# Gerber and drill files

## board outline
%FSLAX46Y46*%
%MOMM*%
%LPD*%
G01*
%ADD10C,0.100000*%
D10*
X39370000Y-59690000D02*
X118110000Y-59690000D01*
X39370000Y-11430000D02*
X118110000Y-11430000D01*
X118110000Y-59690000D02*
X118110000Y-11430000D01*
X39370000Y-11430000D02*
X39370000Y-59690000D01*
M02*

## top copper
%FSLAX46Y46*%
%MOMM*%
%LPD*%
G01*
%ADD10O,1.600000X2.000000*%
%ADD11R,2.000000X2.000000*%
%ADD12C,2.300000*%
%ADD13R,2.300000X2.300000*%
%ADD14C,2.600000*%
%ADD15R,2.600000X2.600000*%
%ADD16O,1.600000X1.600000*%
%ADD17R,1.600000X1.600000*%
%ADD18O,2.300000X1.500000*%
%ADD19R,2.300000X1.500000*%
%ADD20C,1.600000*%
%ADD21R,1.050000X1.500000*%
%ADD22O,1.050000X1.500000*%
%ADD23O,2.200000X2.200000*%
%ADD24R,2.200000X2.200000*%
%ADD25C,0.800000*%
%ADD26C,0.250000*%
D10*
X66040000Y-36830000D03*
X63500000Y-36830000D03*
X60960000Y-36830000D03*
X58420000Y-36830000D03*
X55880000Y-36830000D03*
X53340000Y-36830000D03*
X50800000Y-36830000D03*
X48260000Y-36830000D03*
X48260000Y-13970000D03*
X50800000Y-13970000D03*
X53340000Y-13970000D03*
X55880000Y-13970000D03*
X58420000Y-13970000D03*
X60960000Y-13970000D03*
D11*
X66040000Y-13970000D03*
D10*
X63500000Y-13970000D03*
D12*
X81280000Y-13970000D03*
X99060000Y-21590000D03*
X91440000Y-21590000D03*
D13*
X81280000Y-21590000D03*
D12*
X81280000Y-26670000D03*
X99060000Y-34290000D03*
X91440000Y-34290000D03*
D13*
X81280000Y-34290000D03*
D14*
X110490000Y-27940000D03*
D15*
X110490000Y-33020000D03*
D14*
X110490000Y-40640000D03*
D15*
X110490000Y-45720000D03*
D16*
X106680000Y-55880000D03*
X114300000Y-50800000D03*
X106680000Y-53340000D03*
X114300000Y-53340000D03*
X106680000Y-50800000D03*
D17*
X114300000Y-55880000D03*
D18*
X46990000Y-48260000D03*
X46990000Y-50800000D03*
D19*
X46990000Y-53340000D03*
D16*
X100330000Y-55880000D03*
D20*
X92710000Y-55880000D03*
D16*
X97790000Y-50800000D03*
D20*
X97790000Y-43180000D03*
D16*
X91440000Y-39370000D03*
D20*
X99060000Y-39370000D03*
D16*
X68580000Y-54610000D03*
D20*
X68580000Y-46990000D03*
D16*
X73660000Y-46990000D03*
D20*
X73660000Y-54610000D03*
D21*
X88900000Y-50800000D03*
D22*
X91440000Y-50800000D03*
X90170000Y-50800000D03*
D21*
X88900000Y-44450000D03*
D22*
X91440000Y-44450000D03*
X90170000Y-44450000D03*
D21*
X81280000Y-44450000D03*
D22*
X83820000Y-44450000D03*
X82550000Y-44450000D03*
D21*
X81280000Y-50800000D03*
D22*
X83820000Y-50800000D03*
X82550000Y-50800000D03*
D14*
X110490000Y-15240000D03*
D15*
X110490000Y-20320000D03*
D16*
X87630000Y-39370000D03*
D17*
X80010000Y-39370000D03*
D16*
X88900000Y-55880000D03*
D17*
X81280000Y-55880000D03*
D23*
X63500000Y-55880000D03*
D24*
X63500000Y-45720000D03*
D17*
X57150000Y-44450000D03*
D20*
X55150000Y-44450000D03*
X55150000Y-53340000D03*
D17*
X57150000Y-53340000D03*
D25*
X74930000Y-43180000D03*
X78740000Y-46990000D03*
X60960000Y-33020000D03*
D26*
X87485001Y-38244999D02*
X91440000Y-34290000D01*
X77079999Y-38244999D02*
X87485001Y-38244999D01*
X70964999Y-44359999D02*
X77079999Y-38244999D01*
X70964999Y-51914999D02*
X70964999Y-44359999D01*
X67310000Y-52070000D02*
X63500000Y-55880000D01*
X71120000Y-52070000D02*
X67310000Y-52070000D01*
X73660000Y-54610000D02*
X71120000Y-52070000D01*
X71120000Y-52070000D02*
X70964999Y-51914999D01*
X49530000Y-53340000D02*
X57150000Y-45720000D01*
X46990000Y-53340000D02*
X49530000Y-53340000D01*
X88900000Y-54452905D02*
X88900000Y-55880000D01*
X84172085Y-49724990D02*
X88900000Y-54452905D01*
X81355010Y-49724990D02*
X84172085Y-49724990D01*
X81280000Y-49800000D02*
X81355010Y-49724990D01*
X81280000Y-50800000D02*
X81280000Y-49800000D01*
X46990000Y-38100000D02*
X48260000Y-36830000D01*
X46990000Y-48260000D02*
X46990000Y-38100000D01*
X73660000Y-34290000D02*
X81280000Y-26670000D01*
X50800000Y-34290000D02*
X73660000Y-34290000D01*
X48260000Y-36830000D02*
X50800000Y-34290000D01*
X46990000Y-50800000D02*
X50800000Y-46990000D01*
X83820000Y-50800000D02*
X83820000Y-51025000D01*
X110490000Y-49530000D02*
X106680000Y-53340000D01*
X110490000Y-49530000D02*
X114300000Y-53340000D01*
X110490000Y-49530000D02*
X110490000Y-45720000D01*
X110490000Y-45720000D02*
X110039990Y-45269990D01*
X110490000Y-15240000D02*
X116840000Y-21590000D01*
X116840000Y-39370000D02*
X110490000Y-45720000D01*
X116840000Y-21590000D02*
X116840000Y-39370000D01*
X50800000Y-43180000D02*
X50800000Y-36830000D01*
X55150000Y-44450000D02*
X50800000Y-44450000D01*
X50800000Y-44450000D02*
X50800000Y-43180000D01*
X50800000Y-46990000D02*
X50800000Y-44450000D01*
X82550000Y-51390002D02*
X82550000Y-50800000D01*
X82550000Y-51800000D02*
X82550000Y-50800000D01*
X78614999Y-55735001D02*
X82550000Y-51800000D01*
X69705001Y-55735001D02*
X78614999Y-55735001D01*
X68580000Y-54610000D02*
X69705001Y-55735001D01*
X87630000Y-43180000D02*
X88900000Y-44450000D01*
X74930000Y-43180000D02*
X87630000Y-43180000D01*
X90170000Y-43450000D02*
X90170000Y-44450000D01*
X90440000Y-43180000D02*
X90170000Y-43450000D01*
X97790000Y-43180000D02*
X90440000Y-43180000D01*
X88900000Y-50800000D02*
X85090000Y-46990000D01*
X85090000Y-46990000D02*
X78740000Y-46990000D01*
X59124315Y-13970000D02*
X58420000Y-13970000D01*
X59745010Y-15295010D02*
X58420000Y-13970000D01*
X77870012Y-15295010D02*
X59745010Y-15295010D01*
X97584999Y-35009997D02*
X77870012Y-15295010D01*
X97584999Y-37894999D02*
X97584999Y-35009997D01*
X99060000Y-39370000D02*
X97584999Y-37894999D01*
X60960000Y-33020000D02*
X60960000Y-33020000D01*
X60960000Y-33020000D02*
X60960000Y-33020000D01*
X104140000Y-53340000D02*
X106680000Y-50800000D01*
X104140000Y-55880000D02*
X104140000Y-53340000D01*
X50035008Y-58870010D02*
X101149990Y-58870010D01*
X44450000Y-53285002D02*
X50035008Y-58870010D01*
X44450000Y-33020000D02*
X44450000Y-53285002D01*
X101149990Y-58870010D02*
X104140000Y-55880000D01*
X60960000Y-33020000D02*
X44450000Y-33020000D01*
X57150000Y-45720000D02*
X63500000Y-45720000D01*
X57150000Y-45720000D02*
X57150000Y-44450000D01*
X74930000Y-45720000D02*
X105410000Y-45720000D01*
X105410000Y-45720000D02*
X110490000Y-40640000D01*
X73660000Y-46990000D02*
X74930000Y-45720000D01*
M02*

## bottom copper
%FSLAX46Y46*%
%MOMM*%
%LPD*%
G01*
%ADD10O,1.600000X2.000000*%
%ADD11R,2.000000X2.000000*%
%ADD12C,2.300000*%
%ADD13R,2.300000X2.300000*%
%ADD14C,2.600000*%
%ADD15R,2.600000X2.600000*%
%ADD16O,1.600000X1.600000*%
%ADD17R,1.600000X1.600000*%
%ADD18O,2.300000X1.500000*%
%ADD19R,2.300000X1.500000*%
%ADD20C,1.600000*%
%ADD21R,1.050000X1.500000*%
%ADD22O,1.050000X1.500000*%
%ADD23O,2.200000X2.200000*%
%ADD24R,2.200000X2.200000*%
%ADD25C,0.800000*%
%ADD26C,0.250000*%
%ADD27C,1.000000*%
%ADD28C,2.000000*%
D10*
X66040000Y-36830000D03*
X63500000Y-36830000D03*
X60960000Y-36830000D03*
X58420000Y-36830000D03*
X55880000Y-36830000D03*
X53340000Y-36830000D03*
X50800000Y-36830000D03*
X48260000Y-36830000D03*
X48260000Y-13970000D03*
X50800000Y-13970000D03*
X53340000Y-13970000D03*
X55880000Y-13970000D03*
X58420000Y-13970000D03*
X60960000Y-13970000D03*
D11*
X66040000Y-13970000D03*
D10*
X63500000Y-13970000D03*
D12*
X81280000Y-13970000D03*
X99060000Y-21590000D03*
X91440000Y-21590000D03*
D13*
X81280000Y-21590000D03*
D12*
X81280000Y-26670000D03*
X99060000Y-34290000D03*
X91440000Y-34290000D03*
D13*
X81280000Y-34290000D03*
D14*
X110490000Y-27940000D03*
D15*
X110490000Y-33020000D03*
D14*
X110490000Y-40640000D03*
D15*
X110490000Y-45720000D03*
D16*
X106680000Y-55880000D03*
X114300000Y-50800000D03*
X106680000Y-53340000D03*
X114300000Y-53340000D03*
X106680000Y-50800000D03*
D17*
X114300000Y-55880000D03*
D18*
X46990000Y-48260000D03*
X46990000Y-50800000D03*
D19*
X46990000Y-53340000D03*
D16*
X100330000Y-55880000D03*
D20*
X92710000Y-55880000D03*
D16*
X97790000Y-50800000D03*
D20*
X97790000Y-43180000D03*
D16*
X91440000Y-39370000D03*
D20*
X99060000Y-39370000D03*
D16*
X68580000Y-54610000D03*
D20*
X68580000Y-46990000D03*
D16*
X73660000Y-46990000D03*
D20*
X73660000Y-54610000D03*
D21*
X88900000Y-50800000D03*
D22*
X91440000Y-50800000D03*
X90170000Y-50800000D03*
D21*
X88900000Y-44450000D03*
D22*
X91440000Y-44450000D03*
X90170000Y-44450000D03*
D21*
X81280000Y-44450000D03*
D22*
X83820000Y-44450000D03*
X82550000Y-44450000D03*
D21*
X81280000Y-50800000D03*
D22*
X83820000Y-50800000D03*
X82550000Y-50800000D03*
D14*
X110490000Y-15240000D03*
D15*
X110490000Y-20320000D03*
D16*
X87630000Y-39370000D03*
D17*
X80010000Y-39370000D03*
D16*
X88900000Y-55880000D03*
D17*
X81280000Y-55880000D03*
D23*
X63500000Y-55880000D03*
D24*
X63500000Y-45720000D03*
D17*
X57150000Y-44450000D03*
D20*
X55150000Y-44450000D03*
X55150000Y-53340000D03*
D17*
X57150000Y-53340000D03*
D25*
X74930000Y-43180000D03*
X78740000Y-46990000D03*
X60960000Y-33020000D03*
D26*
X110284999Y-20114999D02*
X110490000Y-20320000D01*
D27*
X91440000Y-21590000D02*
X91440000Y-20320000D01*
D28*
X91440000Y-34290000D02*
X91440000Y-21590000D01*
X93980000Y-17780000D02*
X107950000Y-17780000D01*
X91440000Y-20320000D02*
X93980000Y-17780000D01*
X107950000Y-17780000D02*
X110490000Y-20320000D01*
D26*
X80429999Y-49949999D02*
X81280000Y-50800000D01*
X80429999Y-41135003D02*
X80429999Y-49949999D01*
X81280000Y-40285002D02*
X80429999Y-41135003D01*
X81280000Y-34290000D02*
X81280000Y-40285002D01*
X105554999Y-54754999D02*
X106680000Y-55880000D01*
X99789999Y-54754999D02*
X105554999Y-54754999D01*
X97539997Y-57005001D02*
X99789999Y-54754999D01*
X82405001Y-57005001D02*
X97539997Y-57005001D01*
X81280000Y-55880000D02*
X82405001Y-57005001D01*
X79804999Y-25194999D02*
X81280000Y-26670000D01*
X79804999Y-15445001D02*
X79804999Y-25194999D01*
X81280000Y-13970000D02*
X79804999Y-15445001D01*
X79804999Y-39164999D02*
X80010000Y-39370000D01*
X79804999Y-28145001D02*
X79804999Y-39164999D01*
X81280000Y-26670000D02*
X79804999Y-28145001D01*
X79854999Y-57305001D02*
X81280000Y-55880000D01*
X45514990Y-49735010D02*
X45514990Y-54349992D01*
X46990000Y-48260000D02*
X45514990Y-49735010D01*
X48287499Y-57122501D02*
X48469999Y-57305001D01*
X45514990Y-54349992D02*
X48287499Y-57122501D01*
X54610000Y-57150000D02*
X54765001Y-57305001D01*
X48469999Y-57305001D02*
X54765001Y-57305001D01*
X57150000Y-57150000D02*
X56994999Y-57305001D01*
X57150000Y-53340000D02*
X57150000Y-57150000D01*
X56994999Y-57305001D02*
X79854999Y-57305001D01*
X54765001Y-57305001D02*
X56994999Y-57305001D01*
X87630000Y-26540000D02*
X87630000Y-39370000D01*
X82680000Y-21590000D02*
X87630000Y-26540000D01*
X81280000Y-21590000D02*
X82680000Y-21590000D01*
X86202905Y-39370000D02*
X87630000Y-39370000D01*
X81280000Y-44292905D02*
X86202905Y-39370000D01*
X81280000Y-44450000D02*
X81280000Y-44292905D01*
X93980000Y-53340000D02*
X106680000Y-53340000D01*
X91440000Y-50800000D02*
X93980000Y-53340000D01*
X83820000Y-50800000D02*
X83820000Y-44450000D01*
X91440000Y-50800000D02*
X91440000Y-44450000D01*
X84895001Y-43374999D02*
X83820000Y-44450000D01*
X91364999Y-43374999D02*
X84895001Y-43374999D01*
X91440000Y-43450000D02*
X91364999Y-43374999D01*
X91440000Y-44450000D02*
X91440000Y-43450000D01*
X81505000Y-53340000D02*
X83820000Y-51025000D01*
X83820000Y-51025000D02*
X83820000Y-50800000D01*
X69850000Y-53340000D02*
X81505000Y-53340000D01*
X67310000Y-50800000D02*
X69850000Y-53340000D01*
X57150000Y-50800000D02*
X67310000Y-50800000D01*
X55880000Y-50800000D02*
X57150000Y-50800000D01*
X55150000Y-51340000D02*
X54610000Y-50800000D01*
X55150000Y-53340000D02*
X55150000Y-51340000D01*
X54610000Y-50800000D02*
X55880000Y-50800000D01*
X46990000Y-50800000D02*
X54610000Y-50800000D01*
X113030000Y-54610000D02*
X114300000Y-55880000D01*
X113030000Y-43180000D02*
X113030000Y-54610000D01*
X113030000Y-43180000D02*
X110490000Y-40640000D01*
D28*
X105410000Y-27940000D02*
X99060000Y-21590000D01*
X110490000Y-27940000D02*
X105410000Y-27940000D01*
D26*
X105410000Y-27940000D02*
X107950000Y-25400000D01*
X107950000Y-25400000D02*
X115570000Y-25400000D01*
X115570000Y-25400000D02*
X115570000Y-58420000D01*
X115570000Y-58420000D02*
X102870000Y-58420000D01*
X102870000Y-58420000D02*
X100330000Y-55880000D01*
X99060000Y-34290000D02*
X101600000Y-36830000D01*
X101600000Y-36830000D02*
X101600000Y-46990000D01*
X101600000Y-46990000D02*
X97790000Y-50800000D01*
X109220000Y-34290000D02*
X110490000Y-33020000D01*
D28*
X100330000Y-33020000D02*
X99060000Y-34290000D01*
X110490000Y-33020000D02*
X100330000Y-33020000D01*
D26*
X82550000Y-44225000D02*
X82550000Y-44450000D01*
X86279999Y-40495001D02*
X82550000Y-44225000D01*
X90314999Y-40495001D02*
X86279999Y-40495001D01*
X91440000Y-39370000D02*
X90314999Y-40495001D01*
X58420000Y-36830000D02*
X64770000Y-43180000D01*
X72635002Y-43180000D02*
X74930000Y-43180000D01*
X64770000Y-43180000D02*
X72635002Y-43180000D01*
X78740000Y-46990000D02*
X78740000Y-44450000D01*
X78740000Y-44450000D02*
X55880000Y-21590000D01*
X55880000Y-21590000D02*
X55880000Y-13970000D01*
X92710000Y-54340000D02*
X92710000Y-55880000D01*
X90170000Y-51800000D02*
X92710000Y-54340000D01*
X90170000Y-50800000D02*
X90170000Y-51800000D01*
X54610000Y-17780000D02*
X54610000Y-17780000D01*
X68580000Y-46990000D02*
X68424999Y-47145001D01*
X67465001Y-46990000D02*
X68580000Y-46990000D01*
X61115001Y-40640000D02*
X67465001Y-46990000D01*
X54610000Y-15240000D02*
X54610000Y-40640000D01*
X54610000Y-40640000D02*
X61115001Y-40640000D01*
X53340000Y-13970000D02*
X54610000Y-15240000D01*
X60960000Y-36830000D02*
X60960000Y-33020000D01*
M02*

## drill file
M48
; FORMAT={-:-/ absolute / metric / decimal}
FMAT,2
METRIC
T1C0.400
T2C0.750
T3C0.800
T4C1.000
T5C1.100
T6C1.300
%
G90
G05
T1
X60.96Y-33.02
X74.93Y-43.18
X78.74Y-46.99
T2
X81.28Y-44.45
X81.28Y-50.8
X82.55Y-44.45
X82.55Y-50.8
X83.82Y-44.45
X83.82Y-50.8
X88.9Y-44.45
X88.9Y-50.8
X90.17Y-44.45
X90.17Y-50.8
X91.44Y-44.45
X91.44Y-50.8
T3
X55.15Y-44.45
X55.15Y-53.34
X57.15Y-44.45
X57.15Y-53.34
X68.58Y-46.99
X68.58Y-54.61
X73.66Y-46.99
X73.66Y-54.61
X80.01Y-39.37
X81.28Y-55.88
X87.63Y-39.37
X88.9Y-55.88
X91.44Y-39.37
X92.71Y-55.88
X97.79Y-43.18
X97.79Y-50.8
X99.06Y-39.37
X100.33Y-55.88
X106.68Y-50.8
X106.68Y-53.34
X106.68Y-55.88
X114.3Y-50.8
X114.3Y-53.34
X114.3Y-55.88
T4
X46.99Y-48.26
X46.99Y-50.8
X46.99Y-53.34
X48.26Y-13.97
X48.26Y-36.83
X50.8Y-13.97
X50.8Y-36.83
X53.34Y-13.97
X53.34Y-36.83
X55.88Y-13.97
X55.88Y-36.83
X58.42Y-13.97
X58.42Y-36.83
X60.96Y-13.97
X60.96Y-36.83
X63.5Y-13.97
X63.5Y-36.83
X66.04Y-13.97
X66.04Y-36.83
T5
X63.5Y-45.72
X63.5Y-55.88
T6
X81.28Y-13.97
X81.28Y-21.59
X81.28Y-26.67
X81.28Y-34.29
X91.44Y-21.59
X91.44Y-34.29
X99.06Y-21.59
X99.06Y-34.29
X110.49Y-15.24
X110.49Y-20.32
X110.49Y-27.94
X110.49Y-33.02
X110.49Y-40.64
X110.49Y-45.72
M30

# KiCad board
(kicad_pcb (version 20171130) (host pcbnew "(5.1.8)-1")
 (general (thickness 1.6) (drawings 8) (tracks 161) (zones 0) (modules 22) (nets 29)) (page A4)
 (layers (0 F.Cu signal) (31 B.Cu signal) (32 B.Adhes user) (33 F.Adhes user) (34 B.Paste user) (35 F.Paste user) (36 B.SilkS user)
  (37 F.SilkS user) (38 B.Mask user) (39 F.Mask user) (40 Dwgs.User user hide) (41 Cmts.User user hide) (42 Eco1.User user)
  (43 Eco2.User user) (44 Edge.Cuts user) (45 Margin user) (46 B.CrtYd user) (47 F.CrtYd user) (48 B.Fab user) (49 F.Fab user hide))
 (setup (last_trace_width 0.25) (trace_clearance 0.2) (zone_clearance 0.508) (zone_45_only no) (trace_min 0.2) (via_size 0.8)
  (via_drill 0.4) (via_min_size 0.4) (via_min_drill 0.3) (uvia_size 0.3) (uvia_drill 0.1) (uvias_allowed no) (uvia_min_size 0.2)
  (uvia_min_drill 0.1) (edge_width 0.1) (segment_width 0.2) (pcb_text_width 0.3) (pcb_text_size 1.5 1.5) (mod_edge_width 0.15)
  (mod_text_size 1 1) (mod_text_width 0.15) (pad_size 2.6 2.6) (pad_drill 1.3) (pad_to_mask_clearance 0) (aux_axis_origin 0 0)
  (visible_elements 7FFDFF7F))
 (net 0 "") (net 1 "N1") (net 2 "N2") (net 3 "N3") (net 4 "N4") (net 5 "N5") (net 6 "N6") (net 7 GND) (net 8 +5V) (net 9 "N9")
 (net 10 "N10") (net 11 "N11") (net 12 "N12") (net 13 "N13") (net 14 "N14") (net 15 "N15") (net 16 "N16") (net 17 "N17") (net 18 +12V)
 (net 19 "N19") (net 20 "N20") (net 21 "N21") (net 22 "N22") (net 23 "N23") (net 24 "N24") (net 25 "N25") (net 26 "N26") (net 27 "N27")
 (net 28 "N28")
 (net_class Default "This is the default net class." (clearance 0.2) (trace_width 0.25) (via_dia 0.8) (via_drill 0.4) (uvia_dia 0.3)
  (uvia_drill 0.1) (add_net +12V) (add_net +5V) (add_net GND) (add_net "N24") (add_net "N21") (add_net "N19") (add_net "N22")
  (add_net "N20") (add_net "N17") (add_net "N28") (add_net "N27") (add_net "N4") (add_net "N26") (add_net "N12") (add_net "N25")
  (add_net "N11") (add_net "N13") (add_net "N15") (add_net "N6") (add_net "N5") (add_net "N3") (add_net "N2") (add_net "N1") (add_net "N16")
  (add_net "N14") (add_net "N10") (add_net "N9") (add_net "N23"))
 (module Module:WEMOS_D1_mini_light (layer F.Cu) (at 66.04 13.97 270)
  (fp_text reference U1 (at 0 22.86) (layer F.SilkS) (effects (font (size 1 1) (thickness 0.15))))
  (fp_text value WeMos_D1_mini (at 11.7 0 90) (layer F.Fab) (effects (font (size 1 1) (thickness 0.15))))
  (pad 16 thru_hole oval (at 22.86 0 270) (size 2 1.6) (drill 1) (layers *.Cu *.Mask) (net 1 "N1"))
  (pad 15 thru_hole oval (at 22.86 2.54 270) (size 2 1.6) (drill 1) (layers *.Cu *.Mask) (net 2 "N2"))
  (pad 14 thru_hole oval (at 22.86 5.08 270) (size 2 1.6) (drill 1) (layers *.Cu *.Mask) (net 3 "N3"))
  (pad 13 thru_hole oval (at 22.86 7.62 270) (size 2 1.6) (drill 1) (layers *.Cu *.Mask) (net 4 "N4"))
  (pad 12 thru_hole oval (at 22.86 10.16 270) (size 2 1.6) (drill 1) (layers *.Cu *.Mask) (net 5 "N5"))
  (pad 11 thru_hole oval (at 22.86 12.7 270) (size 2 1.6) (drill 1) (layers *.Cu *.Mask) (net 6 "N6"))
  (pad 10 thru_hole oval (at 22.86 15.24 270) (size 2 1.6) (drill 1) (layers *.Cu *.Mask) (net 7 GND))
  (pad 9 thru_hole oval (at 22.86 17.78 270) (size 2 1.6) (drill 1) (layers *.Cu *.Mask) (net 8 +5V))
  (pad 8 thru_hole oval (at 0 17.78 270) (size 2 1.6) (drill 1) (layers *.Cu *.Mask) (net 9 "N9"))
  (pad 7 thru_hole oval (at 0 15.24 270) (size 2 1.6) (drill 1) (layers *.Cu *.Mask) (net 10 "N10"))
  (pad 6 thru_hole oval (at 0 12.7 270) (size 2 1.6) (drill 1) (layers *.Cu *.Mask) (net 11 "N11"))
  (pad 5 thru_hole oval (at 0 10.16 270) (size 2 1.6) (drill 1) (layers *.Cu *.Mask) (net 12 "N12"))
  (pad 4 thru_hole oval (at 0 7.62 270) (size 2 1.6) (drill 1) (layers *.Cu *.Mask) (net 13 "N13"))
  (pad 3 thru_hole oval (at 0 5.08 270) (size 2 1.6) (drill 1) (layers *.Cu *.Mask) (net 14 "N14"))
  (pad 1 thru_hole rect (at 0 0 270) (size 2 2) (drill 1) (layers *.Cu *.Mask) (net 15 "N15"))
  (pad 2 thru_hole oval (at 0 2.54 270) (size 2 1.6) (drill 1) (layers *.Cu *.Mask) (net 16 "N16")))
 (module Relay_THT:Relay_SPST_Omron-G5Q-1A (layer F.Cu) (at 81.28 21.59)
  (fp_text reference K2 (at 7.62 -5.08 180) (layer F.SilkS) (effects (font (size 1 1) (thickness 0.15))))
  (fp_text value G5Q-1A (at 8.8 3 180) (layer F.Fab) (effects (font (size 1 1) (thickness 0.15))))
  (pad 5 thru_hole circle (at 0 -7.62 180) (size 2.3 2.3) (drill 1.3) (layers *.Cu *.Mask) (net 8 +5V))
  (pad 3 thru_hole circle (at 17.78 0 180) (size 2.3 2.3) (drill 1.3) (layers *.Cu *.Mask) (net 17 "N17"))
  (pad 2 thru_hole circle (at 10.16 0 180) (size 2.3 2.3) (drill 1.3) (layers *.Cu *.Mask) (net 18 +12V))
  (pad 1 thru_hole rect (at 0 0 180) (size 2.3 2.3) (drill 1.3) (layers *.Cu *.Mask) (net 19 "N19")))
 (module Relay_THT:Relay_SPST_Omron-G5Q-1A (layer F.Cu) (at 81.28 34.29)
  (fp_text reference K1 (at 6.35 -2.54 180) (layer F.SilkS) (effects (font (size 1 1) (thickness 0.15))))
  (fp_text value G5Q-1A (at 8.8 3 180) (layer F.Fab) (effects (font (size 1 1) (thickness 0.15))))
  (pad 5 thru_hole circle (at 0 -7.62 180) (size 2.3 2.3) (drill 1.3) (layers *.Cu *.Mask) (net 8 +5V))
  (pad 3 thru_hole circle (at 17.78 0 180) (size 2.3 2.3) (drill 1.3) (layers *.Cu *.Mask) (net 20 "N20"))
  (pad 2 thru_hole circle (at 10.16 0 180) (size 2.3 2.3) (drill 1.3) (layers *.Cu *.Mask) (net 18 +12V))
  (pad 1 thru_hole rect (at 0 0 180) (size 2.3 2.3) (drill 1.3) (layers *.Cu *.Mask) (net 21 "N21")))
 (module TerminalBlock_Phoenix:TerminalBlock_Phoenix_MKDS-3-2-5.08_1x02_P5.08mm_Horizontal (layer F.Cu) (at 110.49 33.02 90)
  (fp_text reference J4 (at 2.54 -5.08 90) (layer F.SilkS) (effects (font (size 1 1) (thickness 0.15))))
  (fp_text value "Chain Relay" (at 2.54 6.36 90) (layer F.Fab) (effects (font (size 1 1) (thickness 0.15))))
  (pad 2 thru_hole circle (at 5.08 0 90) (size 2.6 2.6) (drill 1.3) (layers *.Cu *.Mask) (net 17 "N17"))
  (pad 1 thru_hole rect (at 0 0 90) (size 2.6 2.6) (drill 1.3) (layers *.Cu *.Mask) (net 20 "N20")))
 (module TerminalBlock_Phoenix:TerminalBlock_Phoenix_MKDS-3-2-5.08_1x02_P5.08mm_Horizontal (layer F.Cu) (at 110.49 45.72 90)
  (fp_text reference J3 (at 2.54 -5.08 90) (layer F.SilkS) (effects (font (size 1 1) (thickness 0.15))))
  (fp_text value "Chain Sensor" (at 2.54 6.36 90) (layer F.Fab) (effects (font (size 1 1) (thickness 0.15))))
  (pad 2 thru_hole circle (at 5.08 0 90) (size 2.6 2.6) (drill 1.3) (layers *.Cu *.Mask) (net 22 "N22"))
  (pad 1 thru_hole rect (at 0 0 90) (size 2.6 2.6) (drill 1.3) (layers *.Cu *.Mask) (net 7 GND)))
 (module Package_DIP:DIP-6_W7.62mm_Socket (layer F.Cu) (at 114.3 55.88 180)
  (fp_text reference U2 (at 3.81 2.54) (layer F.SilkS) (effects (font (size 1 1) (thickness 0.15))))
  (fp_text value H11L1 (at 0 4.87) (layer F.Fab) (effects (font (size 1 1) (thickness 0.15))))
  (pad 6 thru_hole oval (at 7.62 0 180) (size 1.6 1.6) (drill 0.8) (layers *.Cu *.Mask) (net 8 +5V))
  (pad 3 thru_hole oval (at 0 5.08 180) (size 1.6 1.6) (drill 0.8) (layers *.Cu *.Mask) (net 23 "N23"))
  (pad 5 thru_hole oval (at 7.62 2.54 180) (size 1.6 1.6) (drill 0.8) (layers *.Cu *.Mask) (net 7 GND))
  (pad 2 thru_hole oval (at 0 2.54 180) (size 1.6 1.6) (drill 0.8) (layers *.Cu *.Mask) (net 7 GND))
  (pad 4 thru_hole oval (at 7.62 5.08 180) (size 1.6 1.6) (drill 0.8) (layers *.Cu *.Mask) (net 3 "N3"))
  (pad 1 thru_hole rect (at 0 0 180) (size 1.6 1.6) (drill 0.8) (layers *.Cu *.Mask) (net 22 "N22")))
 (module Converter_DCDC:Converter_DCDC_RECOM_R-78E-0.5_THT (layer F.Cu) (at 46.99 53.34 90)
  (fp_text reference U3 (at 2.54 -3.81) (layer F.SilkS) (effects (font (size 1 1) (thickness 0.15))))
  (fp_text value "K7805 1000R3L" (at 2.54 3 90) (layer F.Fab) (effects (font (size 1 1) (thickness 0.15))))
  (pad 3 thru_hole oval (at 5.08 0 90) (size 1.5 2.3) (drill 1) (layers *.Cu *.Mask) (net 8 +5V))
  (pad 2 thru_hole oval (at 2.54 0 90) (size 1.5 2.3) (drill 1) (layers *.Cu *.Mask) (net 7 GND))
  (pad 1 thru_hole rect (at 0 0 90) (size 1.5 2.3) (drill 1) (layers *.Cu *.Mask) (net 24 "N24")))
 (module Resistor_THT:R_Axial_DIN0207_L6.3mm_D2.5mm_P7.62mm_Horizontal (layer F.Cu) (at 92.71 55.88)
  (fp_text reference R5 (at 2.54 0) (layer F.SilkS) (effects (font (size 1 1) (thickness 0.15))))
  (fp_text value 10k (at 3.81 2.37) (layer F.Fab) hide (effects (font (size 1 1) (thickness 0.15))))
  (pad 2 thru_hole oval (at 7.62 0) (size 1.6 1.6) (drill 0.8) (layers *.Cu *.Mask) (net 17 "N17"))
  (pad 1 thru_hole circle (at 0 0) (size 1.6 1.6) (drill 0.8) (layers *.Cu *.Mask) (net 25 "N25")))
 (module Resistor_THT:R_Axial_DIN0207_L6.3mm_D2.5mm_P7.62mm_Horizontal (layer F.Cu) (at 97.79 43.18 270)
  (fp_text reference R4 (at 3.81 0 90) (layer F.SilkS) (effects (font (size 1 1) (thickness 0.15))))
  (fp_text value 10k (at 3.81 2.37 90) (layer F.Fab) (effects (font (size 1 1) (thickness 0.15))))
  (pad 2 thru_hole oval (at 7.62 0 270) (size 1.6 1.6) (drill 0.8) (layers *.Cu *.Mask) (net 20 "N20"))
  (pad 1 thru_hole circle (at 0 0 270) (size 1.6 1.6) (drill 0.8) (layers *.Cu *.Mask) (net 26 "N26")))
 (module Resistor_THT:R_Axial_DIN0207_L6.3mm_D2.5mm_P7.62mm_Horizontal (layer F.Cu) (at 99.06 39.37 180)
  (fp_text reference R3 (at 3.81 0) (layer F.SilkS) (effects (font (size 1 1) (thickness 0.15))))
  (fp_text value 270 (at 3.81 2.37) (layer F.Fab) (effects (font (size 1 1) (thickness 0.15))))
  (pad 2 thru_hole oval (at 7.62 0 180) (size 1.6 1.6) (drill 0.8) (layers *.Cu *.Mask) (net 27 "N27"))
  (pad 1 thru_hole circle (at 0 0 180) (size 1.6 1.6) (drill 0.8) (layers *.Cu *.Mask) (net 13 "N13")))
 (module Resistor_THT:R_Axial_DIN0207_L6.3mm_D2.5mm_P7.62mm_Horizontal (layer F.Cu) (at 68.58 46.99 270)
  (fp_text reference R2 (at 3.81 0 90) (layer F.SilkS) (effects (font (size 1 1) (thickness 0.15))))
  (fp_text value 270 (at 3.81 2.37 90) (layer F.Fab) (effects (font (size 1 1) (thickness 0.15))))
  (pad 2 thru_hole oval (at 7.62 0 270) (size 1.6 1.6) (drill 0.8) (layers *.Cu *.Mask) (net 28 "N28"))
  (pad 1 thru_hole circle (at 0 0 270) (size 1.6 1.6) (drill 0.8) (layers *.Cu *.Mask) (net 11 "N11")))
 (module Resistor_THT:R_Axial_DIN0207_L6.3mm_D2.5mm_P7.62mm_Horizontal (layer F.Cu) (at 73.66 54.61 90)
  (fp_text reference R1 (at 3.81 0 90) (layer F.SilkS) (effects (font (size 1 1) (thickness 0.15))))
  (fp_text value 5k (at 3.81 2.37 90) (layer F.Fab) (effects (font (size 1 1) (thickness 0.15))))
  (pad 2 thru_hole oval (at 7.62 0 90) (size 1.6 1.6) (drill 0.8) (layers *.Cu *.Mask) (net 22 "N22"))
  (pad 1 thru_hole circle (at 0 0 90) (size 1.6 1.6) (drill 0.8) (layers *.Cu *.Mask) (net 18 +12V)))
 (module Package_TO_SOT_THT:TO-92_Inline (layer F.Cu) (at 88.9 50.8)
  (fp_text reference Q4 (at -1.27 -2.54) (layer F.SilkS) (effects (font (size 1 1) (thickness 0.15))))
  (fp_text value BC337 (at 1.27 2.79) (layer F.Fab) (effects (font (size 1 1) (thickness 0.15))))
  (pad 1 thru_hole rect (at 0 0) (size 1.05 1.5) (drill 0.75) (layers *.Cu *.Mask) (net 12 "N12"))
  (pad 3 thru_hole oval (at 2.54 0) (size 1.05 1.5) (drill 0.75) (layers *.Cu *.Mask) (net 7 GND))
  (pad 2 thru_hole oval (at 1.27 0) (size 1.05 1.5) (drill 0.75) (layers *.Cu *.Mask) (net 25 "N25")))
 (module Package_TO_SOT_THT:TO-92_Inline (layer F.Cu) (at 88.9 44.45)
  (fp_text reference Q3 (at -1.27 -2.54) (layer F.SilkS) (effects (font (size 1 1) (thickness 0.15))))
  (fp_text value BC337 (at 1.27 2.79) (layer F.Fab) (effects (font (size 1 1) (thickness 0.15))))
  (pad 1 thru_hole rect (at 0 0) (size 1.05 1.5) (drill 0.75) (layers *.Cu *.Mask) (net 4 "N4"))
  (pad 3 thru_hole oval (at 2.54 0) (size 1.05 1.5) (drill 0.75) (layers *.Cu *.Mask) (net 7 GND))
  (pad 2 thru_hole oval (at 1.27 0) (size 1.05 1.5) (drill 0.75) (layers *.Cu *.Mask) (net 26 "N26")))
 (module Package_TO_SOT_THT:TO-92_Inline (layer F.Cu) (at 81.28 44.45)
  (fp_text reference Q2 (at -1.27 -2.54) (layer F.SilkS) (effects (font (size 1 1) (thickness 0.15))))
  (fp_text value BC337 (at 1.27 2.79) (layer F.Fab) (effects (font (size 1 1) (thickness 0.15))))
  (pad 1 thru_hole rect (at 0 0) (size 1.05 1.5) (drill 0.75) (layers *.Cu *.Mask) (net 19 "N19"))
  (pad 3 thru_hole oval (at 2.54 0) (size 1.05 1.5) (drill 0.75) (layers *.Cu *.Mask) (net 7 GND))
  (pad 2 thru_hole oval (at 1.27 0) (size 1.05 1.5) (drill 0.75) (layers *.Cu *.Mask) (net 27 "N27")))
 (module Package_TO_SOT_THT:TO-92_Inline (layer F.Cu) (at 81.28 50.8)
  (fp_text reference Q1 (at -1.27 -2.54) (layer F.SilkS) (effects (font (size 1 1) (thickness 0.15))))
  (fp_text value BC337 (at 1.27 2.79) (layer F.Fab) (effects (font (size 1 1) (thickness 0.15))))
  (pad 1 thru_hole rect (at 0 0) (size 1.05 1.5) (drill 0.75) (layers *.Cu *.Mask) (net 21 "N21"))
  (pad 3 thru_hole oval (at 2.54 0) (size 1.05 1.5) (drill 0.75) (layers *.Cu *.Mask) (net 7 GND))
  (pad 2 thru_hole oval (at 1.27 0) (size 1.05 1.5) (drill 0.75) (layers *.Cu *.Mask) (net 28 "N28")))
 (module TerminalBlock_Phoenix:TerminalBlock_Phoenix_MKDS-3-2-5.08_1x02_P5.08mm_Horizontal (layer F.Cu) (at 110.49 20.32 90)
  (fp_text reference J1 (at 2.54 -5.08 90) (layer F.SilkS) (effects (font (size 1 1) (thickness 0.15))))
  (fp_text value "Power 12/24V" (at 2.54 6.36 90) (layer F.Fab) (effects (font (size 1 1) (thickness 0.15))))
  (pad 2 thru_hole circle (at 5.08 0 90) (size 2.6 2.6) (drill 1.3) (layers *.Cu *.Mask) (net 7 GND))
  (pad 1 thru_hole rect (at 0 0 90) (size 2.6 2.6) (drill 1.3) (layers *.Cu *.Mask) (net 18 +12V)))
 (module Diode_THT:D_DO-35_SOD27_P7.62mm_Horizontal (layer F.Cu) (at 80.01 39.37)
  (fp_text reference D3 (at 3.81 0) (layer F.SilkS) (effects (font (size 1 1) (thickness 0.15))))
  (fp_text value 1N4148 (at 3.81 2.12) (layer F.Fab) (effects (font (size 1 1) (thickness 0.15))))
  (pad 2 thru_hole oval (at 7.62 0) (size 1.6 1.6) (drill 0.8) (layers *.Cu *.Mask) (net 19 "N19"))
  (pad 1 thru_hole rect (at 0 0) (size 1.6 1.6) (drill 0.8) (layers *.Cu *.Mask) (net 8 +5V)))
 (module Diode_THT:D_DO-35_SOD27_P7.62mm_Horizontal (layer F.Cu) (at 81.28 55.88)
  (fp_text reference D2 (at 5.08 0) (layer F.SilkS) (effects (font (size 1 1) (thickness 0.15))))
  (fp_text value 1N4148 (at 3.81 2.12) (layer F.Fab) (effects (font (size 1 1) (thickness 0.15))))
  (pad 2 thru_hole oval (at 7.62 0) (size 1.6 1.6) (drill 0.8) (layers *.Cu *.Mask) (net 21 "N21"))
  (pad 1 thru_hole rect (at 0 0) (size 1.6 1.6) (drill 0.8) (layers *.Cu *.Mask) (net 8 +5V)))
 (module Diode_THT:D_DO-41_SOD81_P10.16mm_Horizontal (layer F.Cu) (at 63.5 45.72 270)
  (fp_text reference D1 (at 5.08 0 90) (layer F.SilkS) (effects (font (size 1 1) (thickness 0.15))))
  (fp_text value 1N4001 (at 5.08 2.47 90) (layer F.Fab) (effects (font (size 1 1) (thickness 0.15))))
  (pad 2 thru_hole oval (at 10.16 0 270) (size 2.2 2.2) (drill 1.1) (layers *.Cu *.Mask) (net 18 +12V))
  (pad 1 thru_hole rect (at 0 0 270) (size 2.2 2.2) (drill 1.1) (layers *.Cu *.Mask) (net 24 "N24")))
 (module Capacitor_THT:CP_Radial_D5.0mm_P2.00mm (layer F.Cu) (at 57.15 44.45 180)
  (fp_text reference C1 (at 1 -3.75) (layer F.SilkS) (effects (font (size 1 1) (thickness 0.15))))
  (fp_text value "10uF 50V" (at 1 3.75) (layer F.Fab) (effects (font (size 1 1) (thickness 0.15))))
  (pad 1 thru_hole rect (at 0 0 180) (size 1.6 1.6) (drill 0.8) (layers *.Cu *.Mask) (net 24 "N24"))
  (pad 2 thru_hole circle (at 2 0 180) (size 1.6 1.6) (drill 0.8) (layers *.Cu *.Mask) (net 7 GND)))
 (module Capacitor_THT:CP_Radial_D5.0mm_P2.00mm (layer F.Cu) (at 57.15 53.34 180)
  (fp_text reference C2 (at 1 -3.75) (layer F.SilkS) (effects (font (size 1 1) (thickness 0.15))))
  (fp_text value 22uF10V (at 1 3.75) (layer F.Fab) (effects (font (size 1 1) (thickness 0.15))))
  (pad 2 thru_hole circle (at 2 0 180) (size 1.6 1.6) (drill 0.8) (layers *.Cu *.Mask) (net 7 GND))
  (pad 1 thru_hole rect (at 0 0 180) (size 1.6 1.6) (drill 0.8) (layers *.Cu *.Mask) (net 8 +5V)))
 (gr_line (start 39.37 59.69) (end 118.11 59.69) (layer Edge.Cuts) (width 0.1))
 (gr_line (start 39.37 11.43) (end 118.11 11.43) (layer Edge.Cuts) (width 0.1))
 (gr_line (start 118.11 59.69) (end 118.11 11.43) (layer Edge.Cuts) (width 0.1))
 (gr_line (start 39.37 11.43) (end 39.37 59.69) (layer Edge.Cuts) (width 0.1))
 (segment (start 110.284999 20.114999) (end 110.49 20.32) (width 0.25) (layer B.Cu) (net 18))
 (segment (start 91.44 21.59) (end 91.44 20.32) (width 1) (layer B.Cu) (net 18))
 (segment (start 91.44 34.29) (end 91.44 21.59) (width 2) (layer B.Cu) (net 18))
 (segment (start 93.98 17.78) (end 107.95 17.78) (width 2) (layer B.Cu) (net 18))
 (segment (start 91.44 20.32) (end 93.98 17.78) (width 2) (layer B.Cu) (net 18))
 (segment (start 87.485001 38.244999) (end 91.44 34.29) (width 0.25) (layer F.Cu) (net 18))
 (segment (start 77.079999 38.244999) (end 87.485001 38.244999) (width 0.25) (layer F.Cu) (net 18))
 (segment (start 70.964999 44.359999) (end 77.079999 38.244999) (width 0.25) (layer F.Cu) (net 18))
 (segment (start 70.964999 51.914999) (end 70.964999 44.359999) (width 0.25) (layer F.Cu) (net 18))
 (segment (start 67.31 52.07) (end 63.5 55.88) (width 0.25) (layer F.Cu) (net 18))
 (segment (start 71.12 52.07) (end 67.31 52.07) (width 0.25) (layer F.Cu) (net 18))
 (segment (start 73.66 54.61) (end 71.12 52.07) (width 0.25) (layer F.Cu) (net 18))
 (segment (start 71.12 52.07) (end 70.964999 51.914999) (width 0.25) (layer F.Cu) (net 18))
 (segment (start 107.95 17.78) (end 110.49 20.32) (width 2) (layer B.Cu) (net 18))
 (segment (start 49.53 53.34) (end 57.15 45.72) (width 0.25) (layer F.Cu) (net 24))
 (segment (start 46.99 53.34) (end 49.53 53.34) (width 0.25) (layer F.Cu) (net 24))
 (segment (start 80.429999 49.949999) (end 81.28 50.8) (width 0.25) (layer B.Cu) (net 21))
 (segment (start 80.429999 41.135003) (end 80.429999 49.949999) (width 0.25) (layer B.Cu) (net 21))
 (segment (start 81.28 40.285002) (end 80.429999 41.135003) (width 0.25) (layer B.Cu) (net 21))
 (segment (start 81.28 34.29) (end 81.28 40.285002) (width 0.25) (layer B.Cu) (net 21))
 (segment (start 88.9 54.452905) (end 88.9 55.88) (width 0.25) (layer F.Cu) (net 21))
 (segment (start 84.172085 49.72499) (end 88.9 54.452905) (width 0.25) (layer F.Cu) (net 21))
 (segment (start 81.35501 49.72499) (end 84.172085 49.72499) (width 0.25) (layer F.Cu) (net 21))
 (segment (start 81.28 49.8) (end 81.35501 49.72499) (width 0.25) (layer F.Cu) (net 21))
 (segment (start 81.28 50.8) (end 81.28 49.8) (width 0.25) (layer F.Cu) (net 21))
 (segment (start 46.99 38.1) (end 48.26 36.83) (width 0.25) (layer F.Cu) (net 8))
 (segment (start 46.99 48.26) (end 46.99 38.1) (width 0.25) (layer F.Cu) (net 8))
 (segment (start 105.554999 54.754999) (end 106.68 55.88) (width 0.25) (layer B.Cu) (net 8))
 (segment (start 99.789999 54.754999) (end 105.554999 54.754999) (width 0.25) (layer B.Cu) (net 8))
 (segment (start 97.539997 57.005001) (end 99.789999 54.754999) (width 0.25) (layer B.Cu) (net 8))
 (segment (start 82.405001 57.005001) (end 97.539997 57.005001) (width 0.25) (layer B.Cu) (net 8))
 (segment (start 81.28 55.88) (end 82.405001 57.005001) (width 0.25) (layer B.Cu) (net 8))
 (segment (start 79.804999 25.194999) (end 81.28 26.67) (width 0.25) (layer B.Cu) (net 8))
 (segment (start 79.804999 15.445001) (end 79.804999 25.194999) (width 0.25) (layer B.Cu) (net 8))
 (segment (start 81.28 13.97) (end 79.804999 15.445001) (width 0.25) (layer B.Cu) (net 8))
 (segment (start 79.804999 39.164999) (end 80.01 39.37) (width 0.25) (layer B.Cu) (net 8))
 (segment (start 79.804999 28.145001) (end 79.804999 39.164999) (width 0.25) (layer B.Cu) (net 8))
 (segment (start 81.28 26.67) (end 79.804999 28.145001) (width 0.25) (layer B.Cu) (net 8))
 (segment (start 79.854999 57.305001) (end 81.28 55.88) (width 0.25) (layer B.Cu) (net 8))
 (segment (start 45.51499 49.73501) (end 45.51499 54.349992) (width 0.25) (layer B.Cu) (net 8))
 (segment (start 46.99 48.26) (end 45.51499 49.73501) (width 0.25) (layer B.Cu) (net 8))
 (segment (start 73.66 34.29) (end 81.28 26.67) (width 0.25) (layer F.Cu) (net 8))
 (segment (start 50.8 34.29) (end 73.66 34.29) (width 0.25) (layer F.Cu) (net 8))
 (segment (start 48.26 36.83) (end 50.8 34.29) (width 0.25) (layer F.Cu) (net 8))
 (segment (start 48.287499 57.122501) (end 48.469999 57.305001) (width 0.25) (layer B.Cu) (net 8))
 (segment (start 45.51499 54.349992) (end 48.287499 57.122501) (width 0.25) (layer B.Cu) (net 8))
 (segment (start 54.61 57.15) (end 54.765001 57.305001) (width 0.25) (layer B.Cu) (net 8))
 (segment (start 48.469999 57.305001) (end 54.765001 57.305001) (width 0.25) (layer B.Cu) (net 8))
 (segment (start 57.15 57.15) (end 56.994999 57.305001) (width 0.25) (layer B.Cu) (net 8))
 (segment (start 57.15 53.34) (end 57.15 57.15) (width 0.25) (layer B.Cu) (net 8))
 (segment (start 56.994999 57.305001) (end 79.854999 57.305001) (width 0.25) (layer B.Cu) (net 8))
 (segment (start 54.765001 57.305001) (end 56.994999 57.305001) (width 0.25) (layer B.Cu) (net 8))
 (segment (start 87.63 26.54) (end 87.63 39.37) (width 0.25) (layer B.Cu) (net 19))
 (segment (start 82.68 21.59) (end 87.63 26.54) (width 0.25) (layer B.Cu) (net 19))
 (segment (start 81.28 21.59) (end 82.68 21.59) (width 0.25) (layer B.Cu) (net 19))
 (segment (start 86.202905 39.37) (end 87.63 39.37) (width 0.25) (layer B.Cu) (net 19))
 (segment (start 81.28 44.292905) (end 86.202905 39.37) (width 0.25) (layer B.Cu) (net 19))
 (segment (start 81.28 44.45) (end 81.28 44.292905) (width 0.25) (layer B.Cu) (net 19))
 (segment (start 46.99 50.8) (end 50.8 46.99) (width 0.25) (layer F.Cu) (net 7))
 (segment (start 83.82 50.8) (end 83.82 51.025) (width 0.25) (layer F.Cu) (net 7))
 (segment (start 110.49 49.53) (end 106.68 53.34) (width 0.25) (layer F.Cu) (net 7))
 (segment (start 110.49 49.53) (end 114.3 53.34) (width 0.25) (layer F.Cu) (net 7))
 (segment (start 110.49 49.53) (end 110.49 45.72) (width 0.25) (layer F.Cu) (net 7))
 (segment (start 110.49 45.72) (end 110.03999 45.26999) (width 0.25) (layer F.Cu) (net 7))
 (segment (start 110.49 15.24) (end 116.84 21.59) (width 0.25) (layer F.Cu) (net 7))
 (segment (start 116.84 39.37) (end 110.49 45.72) (width 0.25) (layer F.Cu) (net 7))
 (segment (start 116.84 21.59) (end 116.84 39.37) (width 0.25) (layer F.Cu) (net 7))
 (segment (start 93.98 53.34) (end 106.68 53.34) (width 0.25) (layer B.Cu) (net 7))
 (segment (start 91.44 50.8) (end 93.98 53.34) (width 0.25) (layer B.Cu) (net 7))
 (segment (start 83.82 50.8) (end 83.82 44.45) (width 0.25) (layer B.Cu) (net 7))
 (segment (start 91.44 50.8) (end 91.44 44.45) (width 0.25) (layer B.Cu) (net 7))
 (segment (start 84.895001 43.374999) (end 83.82 44.45) (width 0.25) (layer B.Cu) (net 7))
 (segment (start 91.364999 43.374999) (end 84.895001 43.374999) (width 0.25) (layer B.Cu) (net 7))
 (segment (start 91.44 43.45) (end 91.364999 43.374999) (width 0.25) (layer B.Cu) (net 7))
 (segment (start 91.44 44.45) (end 91.44 43.45) (width 0.25) (layer B.Cu) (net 7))
 (segment (start 81.505 53.34) (end 83.82 51.025) (width 0.25) (layer B.Cu) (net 7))
 (segment (start 83.82 51.025) (end 83.82 50.8) (width 0.25) (layer B.Cu) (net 7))
 (segment (start 69.85 53.34) (end 81.505 53.34) (width 0.25) (layer B.Cu) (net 7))
 (segment (start 67.31 50.8) (end 69.85 53.34) (width 0.25) (layer B.Cu) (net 7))
 (segment (start 50.8 43.18) (end 50.8 36.83) (width 0.25) (layer F.Cu) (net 7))
 (segment (start 55.15 44.45) (end 50.8 44.45) (width 0.25) (layer F.Cu) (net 7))
 (segment (start 50.8 44.45) (end 50.8 43.18) (width 0.25) (layer F.Cu) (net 7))
 (segment (start 50.8 46.99) (end 50.8 44.45) (width 0.25) (layer F.Cu) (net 7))
 (segment (start 57.15 50.8) (end 67.31 50.8) (width 0.25) (layer B.Cu) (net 7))
 (segment (start 55.88 50.8) (end 57.15 50.8) (width 0.25) (layer B.Cu) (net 7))
 (segment (start 55.15 51.34) (end 54.61 50.8) (width 0.25) (layer B.Cu) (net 7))
 (segment (start 55.15 53.34) (end 55.15 51.34) (width 0.25) (layer B.Cu) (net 7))
 (segment (start 54.61 50.8) (end 55.88 50.8) (width 0.25) (layer B.Cu) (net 7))
 (segment (start 46.99 50.8) (end 54.61 50.8) (width 0.25) (layer B.Cu) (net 7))
 (segment (start 113.03 54.61) (end 114.3 55.88) (width 0.25) (layer B.Cu) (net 22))
 (segment (start 113.03 43.18) (end 113.03 54.61) (width 0.25) (layer B.Cu) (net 22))
 (segment (start 113.03 43.18) (end 110.49 40.64) (width 0.25) (layer B.Cu) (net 22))
 (segment (start 105.41 27.94) (end 99.06 21.59) (width 2) (layer B.Cu) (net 17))
 (segment (start 110.49 27.94) (end 105.41 27.94) (width 2) (layer B.Cu) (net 17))
 (segment (start 105.41 27.94) (end 107.95 25.4) (width 0.25) (layer B.Cu) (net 17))
 (segment (start 107.95 25.4) (end 115.57 25.4) (width 0.25) (layer B.Cu) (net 17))
 (segment (start 115.57 25.4) (end 115.57 58.42) (width 0.25) (layer B.Cu) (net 17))
 (segment (start 115.57 58.42) (end 102.87 58.42) (width 0.25) (layer B.Cu) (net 17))
 (segment (start 102.87 58.42) (end 100.33 55.88) (width 0.25) (layer B.Cu) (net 17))
 (segment (start 99.06 34.29) (end 101.6 36.83) (width 0.25) (layer B.Cu) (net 20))
 (segment (start 101.6 36.83) (end 101.6 46.99) (width 0.25) (layer B.Cu) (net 20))
 (segment (start 101.6 46.99) (end 97.79 50.8) (width 0.25) (layer B.Cu) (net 20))
 (segment (start 109.22 34.29) (end 110.49 33.02) (width 0.25) (layer B.Cu) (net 20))
 (segment (start 100.33 33.02) (end 99.06 34.29) (width 2) (layer B.Cu) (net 20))
 (segment (start 110.49 33.02) (end 100.33 33.02) (width 2) (layer B.Cu) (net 20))
 (segment (start 82.55 51.390002) (end 82.55 50.8) (width 0.25) (layer F.Cu) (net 28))
 (segment (start 82.55 51.8) (end 82.55 50.8) (width 0.25) (layer F.Cu) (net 28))
 (segment (start 78.614999 55.735001) (end 82.55 51.8) (width 0.25) (layer F.Cu) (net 28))
 (segment (start 69.705001 55.735001) (end 78.614999 55.735001) (width 0.25) (layer F.Cu) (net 28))
 (segment (start 68.58 54.61) (end 69.705001 55.735001) (width 0.25) (layer F.Cu) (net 28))
 (segment (start 82.55 44.225) (end 82.55 44.45) (width 0.25) (layer B.Cu) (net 27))
 (segment (start 86.279999 40.495001) (end 82.55 44.225) (width 0.25) (layer B.Cu) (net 27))
 (segment (start 90.314999 40.495001) (end 86.279999 40.495001) (width 0.25) (layer B.Cu) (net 27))
 (segment (start 91.44 39.37) (end 90.314999 40.495001) (width 0.25) (layer B.Cu) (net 27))
 (segment (start 58.42 36.83) (end 64.77 43.18) (width 0.25) (layer B.Cu) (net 4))
 (via (at 74.93 43.18) (size 0.8) (drill 0.4) (layers F.Cu B.Cu) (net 4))
 (segment (start 72.635002 43.18) (end 74.93 43.18) (width 0.25) (layer B.Cu) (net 4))
 (segment (start 64.77 43.18) (end 72.635002 43.18) (width 0.25) (layer B.Cu) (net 4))
 (segment (start 87.63 43.18) (end 88.9 44.45) (width 0.25) (layer F.Cu) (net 4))
 (segment (start 74.93 43.18) (end 87.63 43.18) (width 0.25) (layer F.Cu) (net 4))
 (segment (start 90.17 43.45) (end 90.17 44.45) (width 0.25) (layer F.Cu) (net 26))
 (segment (start 90.44 43.18) (end 90.17 43.45) (width 0.25) (layer F.Cu) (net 26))
 (segment (start 97.79 43.18) (end 90.44 43.18) (width 0.25) (layer F.Cu) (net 26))
 (segment (start 88.9 50.8) (end 85.09 46.99) (width 0.25) (layer F.Cu) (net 12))
 (via (at 78.74 46.99) (size 0.8) (drill 0.4) (layers F.Cu B.Cu) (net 12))
 (segment (start 85.09 46.99) (end 78.74 46.99) (width 0.25) (layer F.Cu) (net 12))
 (segment (start 78.74 46.99) (end 78.74 44.45) (width 0.25) (layer B.Cu) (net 12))
 (segment (start 78.74 44.45) (end 55.88 21.59) (width 0.25) (layer B.Cu) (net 12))
 (segment (start 55.88 21.59) (end 55.88 13.97) (width 0.25) (layer B.Cu) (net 12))
 (segment (start 92.71 54.34) (end 92.71 55.88) (width 0.25) (layer B.Cu) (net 25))
 (segment (start 90.17 51.8) (end 92.71 54.34) (width 0.25) (layer B.Cu) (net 25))
 (segment (start 90.17 50.8) (end 90.17 51.8) (width 0.25) (layer B.Cu) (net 25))
 (segment (start 54.61 17.78) (end 54.61 17.78) (width 0.25) (layer B.Cu) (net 11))
 (segment (start 68.58 46.99) (end 68.424999 47.145001) (width 0.25) (layer B.Cu) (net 11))
 (segment (start 67.465001 46.99) (end 68.58 46.99) (width 0.25) (layer B.Cu) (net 11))
 (segment (start 61.115001 40.64) (end 67.465001 46.99) (width 0.25) (layer B.Cu) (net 11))
 (segment (start 54.61 15.24) (end 54.61 40.64) (width 0.25) (layer B.Cu) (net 11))
 (segment (start 54.61 40.64) (end 61.115001 40.64) (width 0.25) (layer B.Cu) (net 11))
 (segment (start 53.34 13.97) (end 54.61 15.24) (width 0.25) (layer B.Cu) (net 11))
 (segment (start 59.124315 13.97) (end 58.42 13.97) (width 0.25) (layer F.Cu) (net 13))
 (segment (start 59.74501 15.29501) (end 58.42 13.97) (width 0.25) (layer F.Cu) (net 13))
 (segment (start 77.870012 15.29501) (end 59.74501 15.29501) (width 0.25) (layer F.Cu) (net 13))
 (segment (start 97.584999 35.009997) (end 77.870012 15.29501) (width 0.25) (layer F.Cu) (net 13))
 (segment (start 97.584999 37.894999) (end 97.584999 35.009997) (width 0.25) (layer F.Cu) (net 13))
 (segment (start 99.06 39.37) (end 97.584999 37.894999) (width 0.25) (layer F.Cu) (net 13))
 (segment (start 60.96 33.02) (end 60.96 33.02) (width 0.25) (layer F.Cu) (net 3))
 (via (at 60.96 33.02) (size 0.8) (drill 0.4) (layers F.Cu B.Cu) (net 3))
 (segment (start 60.96 33.02) (end 60.96 33.02) (width 0.25) (layer F.Cu) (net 3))
 (segment (start 60.96 36.83) (end 60.96 33.02) (width 0.25) (layer B.Cu) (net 3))
 (segment (start 104.14 53.34) (end 106.68 50.8) (width 0.25) (layer F.Cu) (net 3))
 (segment (start 104.14 55.88) (end 104.14 53.34) (width 0.25) (layer F.Cu) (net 3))
 (segment (start 50.035008 58.87001) (end 101.14999 58.87001) (width 0.25) (layer F.Cu) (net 3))
 (segment (start 44.45 53.285002) (end 50.035008 58.87001) (width 0.25) (layer F.Cu) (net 3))
 (segment (start 44.45 33.02) (end 44.45 53.285002) (width 0.25) (layer F.Cu) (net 3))
 (segment (start 101.14999 58.87001) (end 104.14 55.88) (width 0.25) (layer F.Cu) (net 3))
 (segment (start 60.96 33.02) (end 44.45 33.02) (width 0.25) (layer F.Cu) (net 3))
 (segment (start 57.15 45.72) (end 63.5 45.72) (width 0.25) (layer F.Cu) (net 24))
 (segment (start 57.15 45.72) (end 57.15 44.45) (width 0.25) (layer F.Cu) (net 24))
 (segment (start 74.93 45.72) (end 105.41 45.72) (width 0.25) (layer F.Cu) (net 22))
 (segment (start 105.41 45.72) (end 110.49 40.64) (width 0.25) (layer F.Cu) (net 22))
 (segment (start 73.66 46.99) (end 74.93 45.72) (width 0.25) (layer F.Cu) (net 22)))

